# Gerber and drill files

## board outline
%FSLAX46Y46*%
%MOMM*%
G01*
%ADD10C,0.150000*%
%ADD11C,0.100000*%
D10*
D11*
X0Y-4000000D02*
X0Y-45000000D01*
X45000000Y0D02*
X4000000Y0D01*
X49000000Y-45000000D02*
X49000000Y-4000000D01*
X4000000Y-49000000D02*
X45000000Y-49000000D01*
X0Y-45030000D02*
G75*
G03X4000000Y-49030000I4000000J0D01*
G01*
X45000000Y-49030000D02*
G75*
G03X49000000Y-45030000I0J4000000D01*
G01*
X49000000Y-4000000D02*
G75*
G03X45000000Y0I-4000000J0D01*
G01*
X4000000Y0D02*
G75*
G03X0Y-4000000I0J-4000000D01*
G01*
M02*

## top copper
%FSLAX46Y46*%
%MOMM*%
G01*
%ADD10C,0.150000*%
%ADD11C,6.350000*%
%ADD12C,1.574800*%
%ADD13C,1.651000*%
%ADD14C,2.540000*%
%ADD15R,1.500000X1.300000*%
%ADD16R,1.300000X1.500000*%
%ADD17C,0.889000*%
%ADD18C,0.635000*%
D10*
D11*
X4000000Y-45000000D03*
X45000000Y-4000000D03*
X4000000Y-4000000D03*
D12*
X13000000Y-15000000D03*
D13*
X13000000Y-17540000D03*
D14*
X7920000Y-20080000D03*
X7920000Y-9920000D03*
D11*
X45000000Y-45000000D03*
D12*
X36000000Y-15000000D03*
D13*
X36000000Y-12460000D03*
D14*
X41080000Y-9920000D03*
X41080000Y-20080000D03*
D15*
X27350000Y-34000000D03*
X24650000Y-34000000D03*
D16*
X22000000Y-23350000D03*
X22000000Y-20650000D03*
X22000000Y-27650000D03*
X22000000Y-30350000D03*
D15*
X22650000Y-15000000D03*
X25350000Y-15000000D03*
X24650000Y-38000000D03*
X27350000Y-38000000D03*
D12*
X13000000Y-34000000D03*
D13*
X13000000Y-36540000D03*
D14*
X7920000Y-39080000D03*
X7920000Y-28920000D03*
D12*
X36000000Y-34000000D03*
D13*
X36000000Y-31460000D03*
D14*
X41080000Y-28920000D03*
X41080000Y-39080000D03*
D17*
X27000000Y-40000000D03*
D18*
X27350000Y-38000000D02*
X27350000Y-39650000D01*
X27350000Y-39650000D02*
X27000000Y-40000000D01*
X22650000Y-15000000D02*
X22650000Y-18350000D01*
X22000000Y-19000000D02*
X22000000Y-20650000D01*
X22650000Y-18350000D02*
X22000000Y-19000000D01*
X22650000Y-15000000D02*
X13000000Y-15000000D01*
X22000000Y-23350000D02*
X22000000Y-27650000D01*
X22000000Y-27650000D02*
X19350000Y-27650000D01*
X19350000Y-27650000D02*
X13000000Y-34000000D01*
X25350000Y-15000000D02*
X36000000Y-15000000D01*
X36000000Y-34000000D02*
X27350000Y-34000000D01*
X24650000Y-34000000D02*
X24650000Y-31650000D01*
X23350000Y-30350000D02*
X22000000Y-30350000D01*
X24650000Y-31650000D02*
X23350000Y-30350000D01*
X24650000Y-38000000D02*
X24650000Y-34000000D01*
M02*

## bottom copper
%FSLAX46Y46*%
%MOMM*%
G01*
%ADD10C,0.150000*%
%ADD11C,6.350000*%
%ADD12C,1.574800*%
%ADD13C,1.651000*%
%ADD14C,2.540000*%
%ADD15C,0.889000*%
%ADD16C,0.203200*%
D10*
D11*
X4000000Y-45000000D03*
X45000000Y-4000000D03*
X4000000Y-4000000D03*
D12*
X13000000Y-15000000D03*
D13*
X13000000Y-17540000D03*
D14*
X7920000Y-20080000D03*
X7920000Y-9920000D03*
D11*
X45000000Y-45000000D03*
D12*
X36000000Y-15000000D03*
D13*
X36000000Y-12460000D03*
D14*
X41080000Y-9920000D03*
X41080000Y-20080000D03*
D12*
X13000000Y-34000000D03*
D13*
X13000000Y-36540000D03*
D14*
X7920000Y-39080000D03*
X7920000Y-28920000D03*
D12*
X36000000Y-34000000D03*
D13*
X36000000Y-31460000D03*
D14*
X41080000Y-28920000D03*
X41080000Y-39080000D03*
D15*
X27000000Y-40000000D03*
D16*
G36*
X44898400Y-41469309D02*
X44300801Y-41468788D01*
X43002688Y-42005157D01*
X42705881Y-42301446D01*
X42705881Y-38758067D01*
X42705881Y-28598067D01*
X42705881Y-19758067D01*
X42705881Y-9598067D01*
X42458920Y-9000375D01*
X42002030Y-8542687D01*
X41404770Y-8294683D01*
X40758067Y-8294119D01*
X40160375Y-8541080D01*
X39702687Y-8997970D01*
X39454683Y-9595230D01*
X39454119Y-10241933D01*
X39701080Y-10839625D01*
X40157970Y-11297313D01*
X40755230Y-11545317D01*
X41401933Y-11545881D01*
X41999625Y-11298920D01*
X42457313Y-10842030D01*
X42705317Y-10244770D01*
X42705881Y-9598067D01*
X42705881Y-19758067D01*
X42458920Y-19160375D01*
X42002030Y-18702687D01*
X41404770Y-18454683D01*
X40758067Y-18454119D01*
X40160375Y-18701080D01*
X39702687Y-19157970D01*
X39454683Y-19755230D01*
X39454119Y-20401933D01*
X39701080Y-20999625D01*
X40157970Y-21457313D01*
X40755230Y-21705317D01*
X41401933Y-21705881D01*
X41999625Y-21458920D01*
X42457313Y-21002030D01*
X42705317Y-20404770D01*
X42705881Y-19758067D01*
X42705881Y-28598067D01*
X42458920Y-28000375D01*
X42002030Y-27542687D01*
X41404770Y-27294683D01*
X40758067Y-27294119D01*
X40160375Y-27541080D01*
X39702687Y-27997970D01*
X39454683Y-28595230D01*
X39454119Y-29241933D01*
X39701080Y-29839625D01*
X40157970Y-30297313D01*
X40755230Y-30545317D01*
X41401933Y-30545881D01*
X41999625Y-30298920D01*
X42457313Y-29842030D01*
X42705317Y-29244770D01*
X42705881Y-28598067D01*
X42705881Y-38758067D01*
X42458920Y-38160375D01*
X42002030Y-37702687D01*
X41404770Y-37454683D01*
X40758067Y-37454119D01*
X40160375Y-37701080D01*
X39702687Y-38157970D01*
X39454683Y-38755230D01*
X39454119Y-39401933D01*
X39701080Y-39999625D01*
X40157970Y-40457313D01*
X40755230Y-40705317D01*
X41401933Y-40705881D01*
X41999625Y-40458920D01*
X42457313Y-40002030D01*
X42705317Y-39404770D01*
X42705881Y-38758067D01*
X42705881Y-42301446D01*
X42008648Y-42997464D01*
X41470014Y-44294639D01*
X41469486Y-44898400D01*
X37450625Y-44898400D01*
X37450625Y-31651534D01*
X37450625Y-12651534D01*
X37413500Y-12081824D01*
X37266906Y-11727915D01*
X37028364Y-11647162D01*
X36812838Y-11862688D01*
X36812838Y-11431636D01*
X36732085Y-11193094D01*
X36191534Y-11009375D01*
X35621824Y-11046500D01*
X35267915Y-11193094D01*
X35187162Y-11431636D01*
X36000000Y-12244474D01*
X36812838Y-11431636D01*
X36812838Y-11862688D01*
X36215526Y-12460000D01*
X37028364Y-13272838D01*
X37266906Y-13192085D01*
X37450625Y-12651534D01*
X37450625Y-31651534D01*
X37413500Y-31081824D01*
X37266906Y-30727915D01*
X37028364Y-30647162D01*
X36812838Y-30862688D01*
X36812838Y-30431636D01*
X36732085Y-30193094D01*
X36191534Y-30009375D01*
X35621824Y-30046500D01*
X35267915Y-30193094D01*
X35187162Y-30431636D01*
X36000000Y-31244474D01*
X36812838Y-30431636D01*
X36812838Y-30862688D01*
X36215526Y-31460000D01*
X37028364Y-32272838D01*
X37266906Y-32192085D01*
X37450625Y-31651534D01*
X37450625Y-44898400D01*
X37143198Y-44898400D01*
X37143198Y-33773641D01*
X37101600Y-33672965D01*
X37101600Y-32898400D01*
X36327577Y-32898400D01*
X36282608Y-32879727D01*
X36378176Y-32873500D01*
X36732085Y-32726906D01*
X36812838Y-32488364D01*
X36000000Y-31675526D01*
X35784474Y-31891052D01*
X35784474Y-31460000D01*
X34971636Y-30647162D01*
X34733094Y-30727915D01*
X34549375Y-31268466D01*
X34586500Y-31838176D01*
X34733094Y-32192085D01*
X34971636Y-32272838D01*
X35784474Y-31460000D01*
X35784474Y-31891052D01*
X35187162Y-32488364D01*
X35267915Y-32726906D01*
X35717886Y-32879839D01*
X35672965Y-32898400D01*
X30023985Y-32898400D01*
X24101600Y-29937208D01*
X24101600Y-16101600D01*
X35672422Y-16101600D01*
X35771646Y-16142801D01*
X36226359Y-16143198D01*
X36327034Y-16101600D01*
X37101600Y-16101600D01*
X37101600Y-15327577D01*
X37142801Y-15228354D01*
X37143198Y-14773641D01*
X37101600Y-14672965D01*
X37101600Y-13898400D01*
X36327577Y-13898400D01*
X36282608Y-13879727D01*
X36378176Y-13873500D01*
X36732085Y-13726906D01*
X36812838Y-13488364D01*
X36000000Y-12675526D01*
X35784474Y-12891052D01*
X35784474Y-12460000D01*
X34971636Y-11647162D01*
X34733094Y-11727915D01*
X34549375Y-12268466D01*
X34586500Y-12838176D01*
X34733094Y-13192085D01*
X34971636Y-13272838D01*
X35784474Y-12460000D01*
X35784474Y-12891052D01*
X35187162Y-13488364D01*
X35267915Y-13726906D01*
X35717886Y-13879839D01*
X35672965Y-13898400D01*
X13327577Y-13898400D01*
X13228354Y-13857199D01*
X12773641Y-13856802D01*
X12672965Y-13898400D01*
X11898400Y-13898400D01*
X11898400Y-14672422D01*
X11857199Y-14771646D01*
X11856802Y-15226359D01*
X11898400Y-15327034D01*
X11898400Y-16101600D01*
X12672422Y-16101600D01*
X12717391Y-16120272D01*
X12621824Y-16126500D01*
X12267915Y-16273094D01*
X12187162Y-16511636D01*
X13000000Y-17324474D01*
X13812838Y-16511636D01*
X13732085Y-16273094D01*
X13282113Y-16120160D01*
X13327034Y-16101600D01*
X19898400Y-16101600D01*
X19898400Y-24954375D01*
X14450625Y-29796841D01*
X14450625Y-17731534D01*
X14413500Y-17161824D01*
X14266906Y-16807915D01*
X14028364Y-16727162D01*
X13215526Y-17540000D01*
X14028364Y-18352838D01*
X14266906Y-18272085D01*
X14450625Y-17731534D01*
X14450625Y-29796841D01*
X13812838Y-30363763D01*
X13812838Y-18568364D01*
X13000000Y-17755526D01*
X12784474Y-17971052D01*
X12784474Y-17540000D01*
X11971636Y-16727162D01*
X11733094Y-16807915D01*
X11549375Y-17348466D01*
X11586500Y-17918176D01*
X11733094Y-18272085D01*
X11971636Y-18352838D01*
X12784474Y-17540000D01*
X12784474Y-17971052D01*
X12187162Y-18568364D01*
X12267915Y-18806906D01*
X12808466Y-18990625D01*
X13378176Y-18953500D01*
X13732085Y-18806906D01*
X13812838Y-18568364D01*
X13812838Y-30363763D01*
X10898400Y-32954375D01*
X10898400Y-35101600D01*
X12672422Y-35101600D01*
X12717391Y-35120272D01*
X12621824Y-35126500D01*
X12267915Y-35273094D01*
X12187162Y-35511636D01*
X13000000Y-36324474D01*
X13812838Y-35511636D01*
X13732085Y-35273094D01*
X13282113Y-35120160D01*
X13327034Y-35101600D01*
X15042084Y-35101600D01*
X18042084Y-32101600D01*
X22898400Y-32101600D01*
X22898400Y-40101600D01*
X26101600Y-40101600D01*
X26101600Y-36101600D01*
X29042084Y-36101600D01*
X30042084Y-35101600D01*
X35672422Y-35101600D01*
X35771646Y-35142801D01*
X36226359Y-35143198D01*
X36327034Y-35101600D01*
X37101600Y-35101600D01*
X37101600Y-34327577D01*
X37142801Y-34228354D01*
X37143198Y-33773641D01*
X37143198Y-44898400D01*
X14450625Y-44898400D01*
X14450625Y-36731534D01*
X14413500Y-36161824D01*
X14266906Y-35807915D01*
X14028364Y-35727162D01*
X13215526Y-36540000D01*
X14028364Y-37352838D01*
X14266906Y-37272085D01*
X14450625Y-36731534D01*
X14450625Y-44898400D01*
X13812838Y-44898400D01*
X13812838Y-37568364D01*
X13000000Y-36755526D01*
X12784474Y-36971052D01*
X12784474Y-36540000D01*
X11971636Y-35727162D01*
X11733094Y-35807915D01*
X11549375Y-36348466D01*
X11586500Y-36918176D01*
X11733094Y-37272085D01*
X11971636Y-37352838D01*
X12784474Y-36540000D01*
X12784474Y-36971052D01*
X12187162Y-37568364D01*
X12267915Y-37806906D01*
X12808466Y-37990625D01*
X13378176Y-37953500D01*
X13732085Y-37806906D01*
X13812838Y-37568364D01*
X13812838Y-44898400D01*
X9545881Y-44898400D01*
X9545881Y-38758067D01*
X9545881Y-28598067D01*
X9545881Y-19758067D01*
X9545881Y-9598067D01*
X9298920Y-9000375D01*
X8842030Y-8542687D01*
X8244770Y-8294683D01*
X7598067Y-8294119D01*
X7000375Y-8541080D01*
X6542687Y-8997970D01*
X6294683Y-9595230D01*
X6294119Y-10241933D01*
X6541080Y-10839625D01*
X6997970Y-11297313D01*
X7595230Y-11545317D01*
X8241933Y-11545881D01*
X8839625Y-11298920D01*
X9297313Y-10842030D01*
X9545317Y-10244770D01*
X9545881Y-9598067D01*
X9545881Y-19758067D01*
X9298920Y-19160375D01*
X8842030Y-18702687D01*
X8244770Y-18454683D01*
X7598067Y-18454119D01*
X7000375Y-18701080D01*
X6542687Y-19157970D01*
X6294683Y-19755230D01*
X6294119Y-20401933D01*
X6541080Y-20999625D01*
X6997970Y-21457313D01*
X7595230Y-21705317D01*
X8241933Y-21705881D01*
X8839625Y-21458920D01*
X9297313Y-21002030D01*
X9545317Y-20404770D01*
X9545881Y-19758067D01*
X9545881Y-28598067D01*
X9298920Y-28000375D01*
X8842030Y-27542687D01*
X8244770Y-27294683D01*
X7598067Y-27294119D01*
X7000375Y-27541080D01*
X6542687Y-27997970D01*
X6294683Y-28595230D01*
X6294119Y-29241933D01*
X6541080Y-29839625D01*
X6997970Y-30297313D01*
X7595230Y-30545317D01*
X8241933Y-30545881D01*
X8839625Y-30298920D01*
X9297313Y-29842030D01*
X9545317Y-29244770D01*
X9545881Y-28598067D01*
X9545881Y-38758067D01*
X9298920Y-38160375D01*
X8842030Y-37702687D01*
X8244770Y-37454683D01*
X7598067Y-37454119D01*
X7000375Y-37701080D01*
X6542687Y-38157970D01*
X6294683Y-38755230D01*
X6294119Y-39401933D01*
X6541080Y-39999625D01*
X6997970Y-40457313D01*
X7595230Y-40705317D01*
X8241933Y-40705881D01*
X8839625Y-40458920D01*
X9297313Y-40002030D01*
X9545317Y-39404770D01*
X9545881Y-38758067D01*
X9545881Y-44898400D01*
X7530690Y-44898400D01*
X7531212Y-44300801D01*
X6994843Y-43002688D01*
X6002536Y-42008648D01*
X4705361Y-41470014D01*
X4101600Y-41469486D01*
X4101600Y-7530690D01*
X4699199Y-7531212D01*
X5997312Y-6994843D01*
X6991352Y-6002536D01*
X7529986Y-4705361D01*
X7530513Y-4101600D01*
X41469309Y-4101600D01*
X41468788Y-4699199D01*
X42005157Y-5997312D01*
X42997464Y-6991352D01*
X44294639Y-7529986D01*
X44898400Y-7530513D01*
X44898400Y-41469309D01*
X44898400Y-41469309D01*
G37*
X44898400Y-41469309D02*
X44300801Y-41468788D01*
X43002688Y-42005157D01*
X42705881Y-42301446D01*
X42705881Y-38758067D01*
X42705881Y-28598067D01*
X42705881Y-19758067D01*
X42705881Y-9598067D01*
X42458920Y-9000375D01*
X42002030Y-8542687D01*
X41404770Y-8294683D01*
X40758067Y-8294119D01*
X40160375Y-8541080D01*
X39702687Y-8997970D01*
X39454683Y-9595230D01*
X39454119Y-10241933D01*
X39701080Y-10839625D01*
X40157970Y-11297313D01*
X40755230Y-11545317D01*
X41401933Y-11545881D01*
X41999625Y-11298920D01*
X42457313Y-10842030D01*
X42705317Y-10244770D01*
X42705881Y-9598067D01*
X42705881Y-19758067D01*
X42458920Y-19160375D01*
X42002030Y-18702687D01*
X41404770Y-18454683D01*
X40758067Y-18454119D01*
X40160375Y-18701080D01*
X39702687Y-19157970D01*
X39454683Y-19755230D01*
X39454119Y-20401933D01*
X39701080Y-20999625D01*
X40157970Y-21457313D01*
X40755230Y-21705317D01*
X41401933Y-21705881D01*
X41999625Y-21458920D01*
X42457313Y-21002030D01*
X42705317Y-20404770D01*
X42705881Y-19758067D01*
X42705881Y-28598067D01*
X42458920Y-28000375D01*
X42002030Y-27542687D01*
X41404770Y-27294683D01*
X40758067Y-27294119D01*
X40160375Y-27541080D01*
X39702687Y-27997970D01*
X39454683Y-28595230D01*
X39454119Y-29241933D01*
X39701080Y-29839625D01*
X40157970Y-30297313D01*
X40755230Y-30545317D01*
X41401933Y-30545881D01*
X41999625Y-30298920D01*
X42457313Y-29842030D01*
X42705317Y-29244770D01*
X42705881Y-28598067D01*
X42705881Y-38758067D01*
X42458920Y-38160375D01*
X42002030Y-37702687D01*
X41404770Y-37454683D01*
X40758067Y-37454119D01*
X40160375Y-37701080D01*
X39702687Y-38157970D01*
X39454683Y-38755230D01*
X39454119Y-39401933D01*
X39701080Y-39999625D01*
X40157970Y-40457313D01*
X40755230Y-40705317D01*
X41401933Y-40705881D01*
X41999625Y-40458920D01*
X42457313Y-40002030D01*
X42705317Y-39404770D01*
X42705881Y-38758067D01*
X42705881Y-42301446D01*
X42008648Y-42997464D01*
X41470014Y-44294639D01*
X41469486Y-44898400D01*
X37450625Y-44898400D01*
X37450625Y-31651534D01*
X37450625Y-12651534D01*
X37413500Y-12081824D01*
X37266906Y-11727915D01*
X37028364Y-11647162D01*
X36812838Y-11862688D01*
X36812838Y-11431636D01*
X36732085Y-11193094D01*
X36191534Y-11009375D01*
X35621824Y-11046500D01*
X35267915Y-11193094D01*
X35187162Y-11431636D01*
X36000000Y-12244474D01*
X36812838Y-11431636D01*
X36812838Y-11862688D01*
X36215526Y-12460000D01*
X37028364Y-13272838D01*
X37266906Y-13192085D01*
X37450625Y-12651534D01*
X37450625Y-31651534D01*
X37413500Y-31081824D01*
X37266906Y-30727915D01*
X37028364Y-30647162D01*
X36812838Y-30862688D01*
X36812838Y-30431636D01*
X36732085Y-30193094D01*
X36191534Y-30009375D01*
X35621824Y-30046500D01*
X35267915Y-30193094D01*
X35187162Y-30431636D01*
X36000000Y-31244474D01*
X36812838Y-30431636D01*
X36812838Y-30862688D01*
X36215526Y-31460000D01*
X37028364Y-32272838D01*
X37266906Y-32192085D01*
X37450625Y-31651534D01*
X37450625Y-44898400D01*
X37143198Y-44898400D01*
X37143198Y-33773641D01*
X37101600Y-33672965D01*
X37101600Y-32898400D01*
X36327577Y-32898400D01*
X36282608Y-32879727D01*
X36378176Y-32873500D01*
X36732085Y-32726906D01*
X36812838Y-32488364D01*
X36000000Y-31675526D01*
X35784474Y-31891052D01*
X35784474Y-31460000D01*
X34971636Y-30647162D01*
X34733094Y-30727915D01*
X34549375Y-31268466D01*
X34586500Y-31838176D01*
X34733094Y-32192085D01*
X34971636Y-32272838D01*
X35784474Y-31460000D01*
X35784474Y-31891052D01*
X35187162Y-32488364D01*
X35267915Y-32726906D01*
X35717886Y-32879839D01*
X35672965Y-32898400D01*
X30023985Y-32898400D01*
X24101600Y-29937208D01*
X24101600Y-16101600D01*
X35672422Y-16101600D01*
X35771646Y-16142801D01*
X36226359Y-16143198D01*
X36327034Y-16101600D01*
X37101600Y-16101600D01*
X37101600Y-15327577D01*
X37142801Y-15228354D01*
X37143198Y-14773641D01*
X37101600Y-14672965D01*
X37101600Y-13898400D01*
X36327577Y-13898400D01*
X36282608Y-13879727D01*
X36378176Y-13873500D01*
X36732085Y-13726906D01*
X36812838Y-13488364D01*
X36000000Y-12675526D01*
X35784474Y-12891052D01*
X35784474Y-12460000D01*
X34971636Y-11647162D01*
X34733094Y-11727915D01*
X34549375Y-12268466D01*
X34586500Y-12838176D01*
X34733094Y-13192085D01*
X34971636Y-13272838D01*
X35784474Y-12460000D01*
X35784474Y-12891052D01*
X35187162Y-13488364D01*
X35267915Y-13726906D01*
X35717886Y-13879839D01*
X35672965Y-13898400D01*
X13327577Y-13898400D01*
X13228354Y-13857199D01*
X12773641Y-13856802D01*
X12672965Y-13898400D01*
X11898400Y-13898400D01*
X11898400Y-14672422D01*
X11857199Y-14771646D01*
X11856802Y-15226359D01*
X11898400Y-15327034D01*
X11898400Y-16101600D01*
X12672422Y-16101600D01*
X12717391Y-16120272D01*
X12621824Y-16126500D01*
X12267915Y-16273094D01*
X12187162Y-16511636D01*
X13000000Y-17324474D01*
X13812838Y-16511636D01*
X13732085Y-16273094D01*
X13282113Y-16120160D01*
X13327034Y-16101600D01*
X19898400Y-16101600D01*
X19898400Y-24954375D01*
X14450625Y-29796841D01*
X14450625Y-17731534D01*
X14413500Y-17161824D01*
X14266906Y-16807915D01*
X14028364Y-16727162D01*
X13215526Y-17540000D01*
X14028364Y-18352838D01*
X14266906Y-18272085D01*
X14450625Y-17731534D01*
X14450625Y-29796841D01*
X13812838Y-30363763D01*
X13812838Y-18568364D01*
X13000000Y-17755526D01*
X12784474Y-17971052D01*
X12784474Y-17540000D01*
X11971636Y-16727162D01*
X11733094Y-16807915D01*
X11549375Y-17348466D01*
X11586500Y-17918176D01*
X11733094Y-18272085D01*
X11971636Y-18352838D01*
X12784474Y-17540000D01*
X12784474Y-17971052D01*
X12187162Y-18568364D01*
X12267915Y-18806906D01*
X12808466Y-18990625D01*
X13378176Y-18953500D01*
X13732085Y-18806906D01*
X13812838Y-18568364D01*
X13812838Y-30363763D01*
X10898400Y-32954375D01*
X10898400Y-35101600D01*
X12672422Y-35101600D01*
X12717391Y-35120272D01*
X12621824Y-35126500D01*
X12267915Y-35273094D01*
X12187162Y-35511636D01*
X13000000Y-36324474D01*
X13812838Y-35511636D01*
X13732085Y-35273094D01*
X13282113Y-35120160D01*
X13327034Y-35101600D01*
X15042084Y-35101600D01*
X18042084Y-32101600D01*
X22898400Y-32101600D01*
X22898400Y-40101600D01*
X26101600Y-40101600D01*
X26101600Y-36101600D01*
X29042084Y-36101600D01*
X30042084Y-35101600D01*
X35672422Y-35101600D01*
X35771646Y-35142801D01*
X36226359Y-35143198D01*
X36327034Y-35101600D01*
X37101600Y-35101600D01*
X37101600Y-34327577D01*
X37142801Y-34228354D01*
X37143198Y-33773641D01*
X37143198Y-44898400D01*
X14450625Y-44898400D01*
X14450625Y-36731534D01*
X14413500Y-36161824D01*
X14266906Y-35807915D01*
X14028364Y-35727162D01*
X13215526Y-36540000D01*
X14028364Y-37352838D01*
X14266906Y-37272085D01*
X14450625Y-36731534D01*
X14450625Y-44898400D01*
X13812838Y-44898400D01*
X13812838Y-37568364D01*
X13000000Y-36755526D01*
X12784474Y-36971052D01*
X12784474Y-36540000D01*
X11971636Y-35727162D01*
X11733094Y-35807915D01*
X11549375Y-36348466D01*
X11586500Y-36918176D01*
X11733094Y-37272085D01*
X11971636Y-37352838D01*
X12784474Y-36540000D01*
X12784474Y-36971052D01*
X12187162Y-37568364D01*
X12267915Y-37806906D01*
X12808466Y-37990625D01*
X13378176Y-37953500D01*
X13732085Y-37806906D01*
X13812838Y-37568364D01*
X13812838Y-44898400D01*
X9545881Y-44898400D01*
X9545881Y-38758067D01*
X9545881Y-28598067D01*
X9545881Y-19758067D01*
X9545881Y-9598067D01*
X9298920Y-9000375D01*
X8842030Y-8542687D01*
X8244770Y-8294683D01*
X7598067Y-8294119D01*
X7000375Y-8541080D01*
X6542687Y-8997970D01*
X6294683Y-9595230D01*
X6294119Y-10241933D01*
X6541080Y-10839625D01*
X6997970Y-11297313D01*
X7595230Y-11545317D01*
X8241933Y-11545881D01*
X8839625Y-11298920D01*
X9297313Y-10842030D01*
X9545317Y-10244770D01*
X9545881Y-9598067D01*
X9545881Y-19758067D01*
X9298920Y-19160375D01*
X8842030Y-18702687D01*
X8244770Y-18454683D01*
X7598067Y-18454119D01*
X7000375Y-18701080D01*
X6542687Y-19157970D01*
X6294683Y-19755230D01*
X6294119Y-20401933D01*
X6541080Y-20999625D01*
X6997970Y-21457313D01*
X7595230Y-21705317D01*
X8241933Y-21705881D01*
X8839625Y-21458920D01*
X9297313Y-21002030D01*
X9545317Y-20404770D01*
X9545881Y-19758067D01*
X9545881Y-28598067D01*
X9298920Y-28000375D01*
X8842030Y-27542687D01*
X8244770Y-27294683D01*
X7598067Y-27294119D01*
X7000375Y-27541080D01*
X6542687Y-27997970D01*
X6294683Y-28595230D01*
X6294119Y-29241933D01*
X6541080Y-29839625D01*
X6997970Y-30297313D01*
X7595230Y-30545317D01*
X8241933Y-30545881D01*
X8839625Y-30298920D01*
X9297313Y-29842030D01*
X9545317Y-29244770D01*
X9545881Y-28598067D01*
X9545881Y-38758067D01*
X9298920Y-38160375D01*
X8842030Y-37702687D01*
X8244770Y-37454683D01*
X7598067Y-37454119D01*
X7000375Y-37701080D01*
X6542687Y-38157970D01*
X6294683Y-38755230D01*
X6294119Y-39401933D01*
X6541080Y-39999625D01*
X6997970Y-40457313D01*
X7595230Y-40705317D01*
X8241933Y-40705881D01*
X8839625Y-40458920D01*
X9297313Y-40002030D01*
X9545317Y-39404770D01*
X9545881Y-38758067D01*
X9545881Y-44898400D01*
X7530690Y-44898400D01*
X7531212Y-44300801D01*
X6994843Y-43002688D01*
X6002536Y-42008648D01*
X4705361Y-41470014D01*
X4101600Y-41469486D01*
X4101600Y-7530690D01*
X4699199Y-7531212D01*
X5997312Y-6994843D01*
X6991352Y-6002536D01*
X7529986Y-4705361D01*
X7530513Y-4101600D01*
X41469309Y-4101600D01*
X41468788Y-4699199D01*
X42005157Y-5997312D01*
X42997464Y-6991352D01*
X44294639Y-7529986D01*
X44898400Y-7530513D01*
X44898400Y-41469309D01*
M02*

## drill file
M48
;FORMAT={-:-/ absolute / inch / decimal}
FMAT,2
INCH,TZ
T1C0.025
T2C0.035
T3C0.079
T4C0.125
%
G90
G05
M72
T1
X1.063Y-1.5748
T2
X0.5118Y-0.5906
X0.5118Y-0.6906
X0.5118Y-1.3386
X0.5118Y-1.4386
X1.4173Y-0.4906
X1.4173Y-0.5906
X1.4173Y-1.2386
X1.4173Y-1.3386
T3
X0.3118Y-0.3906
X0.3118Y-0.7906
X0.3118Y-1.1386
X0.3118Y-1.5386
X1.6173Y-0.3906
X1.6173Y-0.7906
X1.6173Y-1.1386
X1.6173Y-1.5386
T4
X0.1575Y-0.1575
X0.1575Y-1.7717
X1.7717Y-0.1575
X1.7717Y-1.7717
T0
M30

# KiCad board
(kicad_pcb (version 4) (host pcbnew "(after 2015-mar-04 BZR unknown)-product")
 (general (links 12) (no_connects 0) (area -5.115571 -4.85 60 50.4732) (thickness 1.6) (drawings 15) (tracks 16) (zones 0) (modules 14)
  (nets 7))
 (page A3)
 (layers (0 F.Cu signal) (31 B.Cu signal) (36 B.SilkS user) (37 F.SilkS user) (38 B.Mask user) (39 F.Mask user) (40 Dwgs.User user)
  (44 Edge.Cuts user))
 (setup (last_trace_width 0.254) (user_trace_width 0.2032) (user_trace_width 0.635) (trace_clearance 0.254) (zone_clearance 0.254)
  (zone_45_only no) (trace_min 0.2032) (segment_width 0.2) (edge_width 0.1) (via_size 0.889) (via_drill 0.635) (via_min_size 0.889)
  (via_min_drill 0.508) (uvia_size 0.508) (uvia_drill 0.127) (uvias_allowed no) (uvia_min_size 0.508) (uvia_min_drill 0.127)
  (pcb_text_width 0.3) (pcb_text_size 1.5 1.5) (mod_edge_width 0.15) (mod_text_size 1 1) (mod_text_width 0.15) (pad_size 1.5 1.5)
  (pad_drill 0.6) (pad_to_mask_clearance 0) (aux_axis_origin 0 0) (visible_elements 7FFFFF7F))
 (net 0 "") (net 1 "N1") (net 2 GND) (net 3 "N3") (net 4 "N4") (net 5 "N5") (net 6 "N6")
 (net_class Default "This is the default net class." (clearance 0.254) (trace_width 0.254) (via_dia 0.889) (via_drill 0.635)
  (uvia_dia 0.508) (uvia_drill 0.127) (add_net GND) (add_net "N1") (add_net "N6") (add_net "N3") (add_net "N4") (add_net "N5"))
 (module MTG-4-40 (layer F.Cu) (at 4 45)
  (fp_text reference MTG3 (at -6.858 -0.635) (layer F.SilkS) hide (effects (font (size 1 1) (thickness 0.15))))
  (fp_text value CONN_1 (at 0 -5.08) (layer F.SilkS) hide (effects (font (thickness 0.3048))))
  (pad 1 thru_hole circle (at 0 0) (size 6.35 6.35) (drill 3.175) (layers *.Cu *.Mask F.SilkS)))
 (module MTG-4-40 (layer F.Cu) (at 45 4)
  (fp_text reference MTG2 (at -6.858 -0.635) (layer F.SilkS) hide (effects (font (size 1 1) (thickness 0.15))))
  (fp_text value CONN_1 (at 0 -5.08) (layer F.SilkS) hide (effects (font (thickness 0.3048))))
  (pad 1 thru_hole circle (at 0 0) (size 6.35 6.35) (drill 3.175) (layers *.Cu *.Mask F.SilkS)))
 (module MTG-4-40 (layer F.Cu) (at 4 4)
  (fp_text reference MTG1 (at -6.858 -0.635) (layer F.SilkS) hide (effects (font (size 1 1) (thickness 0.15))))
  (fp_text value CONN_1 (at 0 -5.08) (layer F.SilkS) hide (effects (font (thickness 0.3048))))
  (pad 1 thru_hole circle (at 0 0) (size 6.35 6.35) (drill 3.175) (layers *.Cu *.Mask F.SilkS)))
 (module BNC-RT (layer F.Cu) (at 13 15 90)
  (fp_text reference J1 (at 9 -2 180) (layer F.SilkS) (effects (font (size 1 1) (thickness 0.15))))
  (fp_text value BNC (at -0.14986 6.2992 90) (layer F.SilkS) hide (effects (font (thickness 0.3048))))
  (pad 1 thru_hole circle (at 0 0 90) (size 1.5748 1.5748) (drill 0.889) (layers *.Cu *.Mask F.SilkS) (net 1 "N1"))
  (pad 2 thru_hole circle (at -2.54 0 90) (size 1.651 1.651) (drill 0.889) (layers *.Cu *.Mask F.SilkS) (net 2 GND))
  (pad "" thru_hole circle (at -5.08 -5.08 90) (size 2.54 2.54) (drill 2.00914) (layers *.Cu *.Mask F.SilkS))
  (pad "" thru_hole circle (at 5.08 -5.08 90) (size 2.54 2.54) (drill 2.00914) (layers *.Cu *.Mask F.SilkS)))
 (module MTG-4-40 (layer F.Cu) (at 45 45)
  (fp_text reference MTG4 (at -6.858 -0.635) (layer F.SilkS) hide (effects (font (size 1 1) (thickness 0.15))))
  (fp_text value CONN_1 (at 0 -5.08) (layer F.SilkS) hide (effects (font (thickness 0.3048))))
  (pad 1 thru_hole circle (at 0 0) (size 6.35 6.35) (drill 3.175) (layers *.Cu *.Mask F.SilkS)))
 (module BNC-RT (layer F.Cu) (at 36 15 270)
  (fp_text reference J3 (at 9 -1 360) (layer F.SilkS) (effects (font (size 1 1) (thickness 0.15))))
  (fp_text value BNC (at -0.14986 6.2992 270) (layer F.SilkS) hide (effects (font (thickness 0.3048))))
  (pad 1 thru_hole circle (at 0 0 270) (size 1.5748 1.5748) (drill 0.889) (layers *.Cu *.Mask F.SilkS) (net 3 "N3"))
  (pad 2 thru_hole circle (at -2.54 0 270) (size 1.651 1.651) (drill 0.889) (layers *.Cu *.Mask F.SilkS) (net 2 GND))
  (pad "" thru_hole circle (at -5.08 -5.08 270) (size 2.54 2.54) (drill 2.00914) (layers *.Cu *.Mask F.SilkS))
  (pad "" thru_hole circle (at 5.08 -5.08 270) (size 2.54 2.54) (drill 2.00914) (layers *.Cu *.Mask F.SilkS)))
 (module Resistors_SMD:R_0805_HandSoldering (layer F.Cu) (at 26 34 180)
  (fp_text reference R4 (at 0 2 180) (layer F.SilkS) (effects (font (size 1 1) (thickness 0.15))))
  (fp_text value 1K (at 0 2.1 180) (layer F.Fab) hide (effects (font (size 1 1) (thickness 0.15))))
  (pad 1 smd rect (at -1.35 0 180) (size 1.5 1.3) (layers F.Cu F.Mask) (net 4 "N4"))
  (pad 2 smd rect (at 1.35 0 180) (size 1.5 1.3) (layers F.Cu F.Mask) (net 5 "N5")))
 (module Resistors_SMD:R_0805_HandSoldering (layer F.Cu) (at 22 22 90)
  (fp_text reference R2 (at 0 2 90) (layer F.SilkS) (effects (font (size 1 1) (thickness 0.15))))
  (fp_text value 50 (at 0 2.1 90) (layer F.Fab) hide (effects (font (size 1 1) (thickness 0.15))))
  (pad 1 smd rect (at -1.35 0 90) (size 1.5 1.3) (layers F.Cu F.Mask) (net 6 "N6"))
  (pad 2 smd rect (at 1.35 0 90) (size 1.5 1.3) (layers F.Cu F.Mask) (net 1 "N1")))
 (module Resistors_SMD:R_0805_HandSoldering (layer F.Cu) (at 22 29 270)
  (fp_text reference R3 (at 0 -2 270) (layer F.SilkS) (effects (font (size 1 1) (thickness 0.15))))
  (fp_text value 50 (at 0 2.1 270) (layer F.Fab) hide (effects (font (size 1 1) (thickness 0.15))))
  (pad 1 smd rect (at -1.35 0 270) (size 1.5 1.3) (layers F.Cu F.Mask) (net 6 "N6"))
  (pad 2 smd rect (at 1.35 0 270) (size 1.5 1.3) (layers F.Cu F.Mask) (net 5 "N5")))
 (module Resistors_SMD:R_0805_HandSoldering (layer F.Cu) (at 24 15)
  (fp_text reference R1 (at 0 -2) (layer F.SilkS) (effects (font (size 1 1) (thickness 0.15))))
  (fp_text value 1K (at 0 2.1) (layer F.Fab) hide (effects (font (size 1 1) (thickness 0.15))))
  (pad 1 smd rect (at -1.35 0) (size 1.5 1.3) (layers F.Cu F.Mask) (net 1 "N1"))
  (pad 2 smd rect (at 1.35 0) (size 1.5 1.3) (layers F.Cu F.Mask) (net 3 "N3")))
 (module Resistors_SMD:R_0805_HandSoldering (layer F.Cu) (at 26 38)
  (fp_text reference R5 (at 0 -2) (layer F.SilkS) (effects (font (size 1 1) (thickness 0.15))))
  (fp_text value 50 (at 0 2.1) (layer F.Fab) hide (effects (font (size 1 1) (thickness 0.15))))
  (pad 1 smd rect (at -1.35 0) (size 1.5 1.3) (layers F.Cu F.Mask) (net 5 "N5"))
  (pad 2 smd rect (at 1.35 0) (size 1.5 1.3) (layers F.Cu F.Mask) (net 2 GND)))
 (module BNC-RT (layer F.Cu) (at 13 34 90)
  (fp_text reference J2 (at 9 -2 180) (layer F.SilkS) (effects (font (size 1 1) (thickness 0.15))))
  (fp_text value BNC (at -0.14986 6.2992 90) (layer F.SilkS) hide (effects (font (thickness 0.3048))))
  (pad 1 thru_hole circle (at 0 0 90) (size 1.5748 1.5748) (drill 0.889) (layers *.Cu *.Mask F.SilkS) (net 6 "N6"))
  (pad 2 thru_hole circle (at -2.54 0 90) (size 1.651 1.651) (drill 0.889) (layers *.Cu *.Mask F.SilkS) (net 2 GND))
  (pad "" thru_hole circle (at -5.08 -5.08 90) (size 2.54 2.54) (drill 2.00914) (layers *.Cu *.Mask F.SilkS))
  (pad "" thru_hole circle (at 5.08 -5.08 90) (size 2.54 2.54) (drill 2.00914) (layers *.Cu *.Mask F.SilkS)))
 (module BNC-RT (layer F.Cu) (at 36 34 270)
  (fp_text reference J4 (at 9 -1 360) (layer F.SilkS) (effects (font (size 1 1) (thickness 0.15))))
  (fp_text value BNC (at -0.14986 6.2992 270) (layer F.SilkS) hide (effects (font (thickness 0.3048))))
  (pad 1 thru_hole circle (at 0 0 270) (size 1.5748 1.5748) (drill 0.889) (layers *.Cu *.Mask F.SilkS) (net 4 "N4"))
  (pad 2 thru_hole circle (at -2.54 0 270) (size 1.651 1.651) (drill 0.889) (layers *.Cu *.Mask F.SilkS) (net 2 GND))
  (pad "" thru_hole circle (at -5.08 -5.08 270) (size 2.54 2.54) (drill 2.00914) (layers *.Cu *.Mask F.SilkS))
  (pad "" thru_hole circle (at 5.08 -5.08 270) (size 2.54 2.54) (drill 2.00914) (layers *.Cu *.Mask F.SilkS)))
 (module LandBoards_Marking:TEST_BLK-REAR (layer F.Cu) (at 24 45)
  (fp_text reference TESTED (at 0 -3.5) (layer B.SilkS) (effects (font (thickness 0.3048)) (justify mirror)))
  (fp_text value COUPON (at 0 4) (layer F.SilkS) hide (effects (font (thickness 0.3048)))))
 (gr_line (start 0 4) (end 0 45) (angle 90) (layer Edge.Cuts) (width 0.1))
 (gr_line (start 45 0) (end 4 0) (angle 90) (layer Edge.Cuts) (width 0.1))
 (gr_line (start 49 45) (end 49 4) (angle 90) (layer Edge.Cuts) (width 0.1))
 (gr_line (start 4 49) (end 45 49) (angle 90) (layer Edge.Cuts) (width 0.1))
 (gr_arc (start 4 45.03) (end 4 49.03) (angle 90) (layer Edge.Cuts) (width 0.1))
 (gr_arc (start 45 45.03) (end 49 45.03) (angle 90) (layer Edge.Cuts) (width 0.1))
 (gr_arc (start 45 4) (end 45 0) (angle 90) (layer Edge.Cuts) (width 0.1))
 (gr_arc (start 4 4) (end 0 4) (angle 90) (layer Edge.Cuts) (width 0.1))
 (segment (start 27.35 38) (end 27.35 39.65) (width 0.635) (layer F.Cu) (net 2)) (via (at 27 40) (size 0.889) (layers F.Cu B.Cu) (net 2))
 (segment (start 27.35 39.65) (end 27 40) (width 0.635) (layer F.Cu) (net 2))
 (segment (start 22.65 15) (end 22.65 18.35) (width 0.635) (layer F.Cu) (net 1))
 (segment (start 22 19) (end 22 20.65) (width 0.635) (layer F.Cu) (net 1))
 (segment (start 22.65 18.35) (end 22 19) (width 0.635) (layer F.Cu) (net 1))
 (segment (start 22.65 15) (end 13 15) (width 0.635) (layer F.Cu) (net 1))
 (segment (start 22 23.35) (end 22 27.65) (width 0.635) (layer F.Cu) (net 6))
 (segment (start 22 27.65) (end 19.35 27.65) (width 0.635) (layer F.Cu) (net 6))
 (segment (start 19.35 27.65) (end 13 34) (width 0.635) (layer F.Cu) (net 6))
 (segment (start 25.35 15) (end 36 15) (width 0.635) (layer F.Cu) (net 3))
 (segment (start 36 34) (end 27.35 34) (width 0.635) (layer F.Cu) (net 4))
 (segment (start 24.65 34) (end 24.65 31.65) (width 0.635) (layer F.Cu) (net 5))
 (segment (start 23.35 30.35) (end 22 30.35) (width 0.635) (layer F.Cu) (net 5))
 (segment (start 24.65 31.65) (end 23.35 30.35) (width 0.635) (layer F.Cu) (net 5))
 (segment (start 24.65 38) (end 24.65 34) (width 0.635) (layer F.Cu) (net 5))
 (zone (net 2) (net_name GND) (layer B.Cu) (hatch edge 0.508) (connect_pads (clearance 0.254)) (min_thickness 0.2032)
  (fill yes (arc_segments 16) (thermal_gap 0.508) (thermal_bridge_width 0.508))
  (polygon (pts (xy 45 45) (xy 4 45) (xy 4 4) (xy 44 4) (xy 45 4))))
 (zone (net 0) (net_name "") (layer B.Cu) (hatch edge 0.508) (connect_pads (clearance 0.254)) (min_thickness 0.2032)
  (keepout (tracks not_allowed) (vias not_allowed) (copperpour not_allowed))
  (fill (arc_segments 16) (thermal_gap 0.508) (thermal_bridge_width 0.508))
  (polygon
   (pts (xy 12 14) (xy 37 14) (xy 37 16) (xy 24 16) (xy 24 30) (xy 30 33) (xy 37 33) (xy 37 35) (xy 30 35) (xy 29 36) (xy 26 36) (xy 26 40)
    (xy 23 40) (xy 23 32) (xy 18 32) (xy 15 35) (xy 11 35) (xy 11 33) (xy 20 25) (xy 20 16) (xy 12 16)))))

